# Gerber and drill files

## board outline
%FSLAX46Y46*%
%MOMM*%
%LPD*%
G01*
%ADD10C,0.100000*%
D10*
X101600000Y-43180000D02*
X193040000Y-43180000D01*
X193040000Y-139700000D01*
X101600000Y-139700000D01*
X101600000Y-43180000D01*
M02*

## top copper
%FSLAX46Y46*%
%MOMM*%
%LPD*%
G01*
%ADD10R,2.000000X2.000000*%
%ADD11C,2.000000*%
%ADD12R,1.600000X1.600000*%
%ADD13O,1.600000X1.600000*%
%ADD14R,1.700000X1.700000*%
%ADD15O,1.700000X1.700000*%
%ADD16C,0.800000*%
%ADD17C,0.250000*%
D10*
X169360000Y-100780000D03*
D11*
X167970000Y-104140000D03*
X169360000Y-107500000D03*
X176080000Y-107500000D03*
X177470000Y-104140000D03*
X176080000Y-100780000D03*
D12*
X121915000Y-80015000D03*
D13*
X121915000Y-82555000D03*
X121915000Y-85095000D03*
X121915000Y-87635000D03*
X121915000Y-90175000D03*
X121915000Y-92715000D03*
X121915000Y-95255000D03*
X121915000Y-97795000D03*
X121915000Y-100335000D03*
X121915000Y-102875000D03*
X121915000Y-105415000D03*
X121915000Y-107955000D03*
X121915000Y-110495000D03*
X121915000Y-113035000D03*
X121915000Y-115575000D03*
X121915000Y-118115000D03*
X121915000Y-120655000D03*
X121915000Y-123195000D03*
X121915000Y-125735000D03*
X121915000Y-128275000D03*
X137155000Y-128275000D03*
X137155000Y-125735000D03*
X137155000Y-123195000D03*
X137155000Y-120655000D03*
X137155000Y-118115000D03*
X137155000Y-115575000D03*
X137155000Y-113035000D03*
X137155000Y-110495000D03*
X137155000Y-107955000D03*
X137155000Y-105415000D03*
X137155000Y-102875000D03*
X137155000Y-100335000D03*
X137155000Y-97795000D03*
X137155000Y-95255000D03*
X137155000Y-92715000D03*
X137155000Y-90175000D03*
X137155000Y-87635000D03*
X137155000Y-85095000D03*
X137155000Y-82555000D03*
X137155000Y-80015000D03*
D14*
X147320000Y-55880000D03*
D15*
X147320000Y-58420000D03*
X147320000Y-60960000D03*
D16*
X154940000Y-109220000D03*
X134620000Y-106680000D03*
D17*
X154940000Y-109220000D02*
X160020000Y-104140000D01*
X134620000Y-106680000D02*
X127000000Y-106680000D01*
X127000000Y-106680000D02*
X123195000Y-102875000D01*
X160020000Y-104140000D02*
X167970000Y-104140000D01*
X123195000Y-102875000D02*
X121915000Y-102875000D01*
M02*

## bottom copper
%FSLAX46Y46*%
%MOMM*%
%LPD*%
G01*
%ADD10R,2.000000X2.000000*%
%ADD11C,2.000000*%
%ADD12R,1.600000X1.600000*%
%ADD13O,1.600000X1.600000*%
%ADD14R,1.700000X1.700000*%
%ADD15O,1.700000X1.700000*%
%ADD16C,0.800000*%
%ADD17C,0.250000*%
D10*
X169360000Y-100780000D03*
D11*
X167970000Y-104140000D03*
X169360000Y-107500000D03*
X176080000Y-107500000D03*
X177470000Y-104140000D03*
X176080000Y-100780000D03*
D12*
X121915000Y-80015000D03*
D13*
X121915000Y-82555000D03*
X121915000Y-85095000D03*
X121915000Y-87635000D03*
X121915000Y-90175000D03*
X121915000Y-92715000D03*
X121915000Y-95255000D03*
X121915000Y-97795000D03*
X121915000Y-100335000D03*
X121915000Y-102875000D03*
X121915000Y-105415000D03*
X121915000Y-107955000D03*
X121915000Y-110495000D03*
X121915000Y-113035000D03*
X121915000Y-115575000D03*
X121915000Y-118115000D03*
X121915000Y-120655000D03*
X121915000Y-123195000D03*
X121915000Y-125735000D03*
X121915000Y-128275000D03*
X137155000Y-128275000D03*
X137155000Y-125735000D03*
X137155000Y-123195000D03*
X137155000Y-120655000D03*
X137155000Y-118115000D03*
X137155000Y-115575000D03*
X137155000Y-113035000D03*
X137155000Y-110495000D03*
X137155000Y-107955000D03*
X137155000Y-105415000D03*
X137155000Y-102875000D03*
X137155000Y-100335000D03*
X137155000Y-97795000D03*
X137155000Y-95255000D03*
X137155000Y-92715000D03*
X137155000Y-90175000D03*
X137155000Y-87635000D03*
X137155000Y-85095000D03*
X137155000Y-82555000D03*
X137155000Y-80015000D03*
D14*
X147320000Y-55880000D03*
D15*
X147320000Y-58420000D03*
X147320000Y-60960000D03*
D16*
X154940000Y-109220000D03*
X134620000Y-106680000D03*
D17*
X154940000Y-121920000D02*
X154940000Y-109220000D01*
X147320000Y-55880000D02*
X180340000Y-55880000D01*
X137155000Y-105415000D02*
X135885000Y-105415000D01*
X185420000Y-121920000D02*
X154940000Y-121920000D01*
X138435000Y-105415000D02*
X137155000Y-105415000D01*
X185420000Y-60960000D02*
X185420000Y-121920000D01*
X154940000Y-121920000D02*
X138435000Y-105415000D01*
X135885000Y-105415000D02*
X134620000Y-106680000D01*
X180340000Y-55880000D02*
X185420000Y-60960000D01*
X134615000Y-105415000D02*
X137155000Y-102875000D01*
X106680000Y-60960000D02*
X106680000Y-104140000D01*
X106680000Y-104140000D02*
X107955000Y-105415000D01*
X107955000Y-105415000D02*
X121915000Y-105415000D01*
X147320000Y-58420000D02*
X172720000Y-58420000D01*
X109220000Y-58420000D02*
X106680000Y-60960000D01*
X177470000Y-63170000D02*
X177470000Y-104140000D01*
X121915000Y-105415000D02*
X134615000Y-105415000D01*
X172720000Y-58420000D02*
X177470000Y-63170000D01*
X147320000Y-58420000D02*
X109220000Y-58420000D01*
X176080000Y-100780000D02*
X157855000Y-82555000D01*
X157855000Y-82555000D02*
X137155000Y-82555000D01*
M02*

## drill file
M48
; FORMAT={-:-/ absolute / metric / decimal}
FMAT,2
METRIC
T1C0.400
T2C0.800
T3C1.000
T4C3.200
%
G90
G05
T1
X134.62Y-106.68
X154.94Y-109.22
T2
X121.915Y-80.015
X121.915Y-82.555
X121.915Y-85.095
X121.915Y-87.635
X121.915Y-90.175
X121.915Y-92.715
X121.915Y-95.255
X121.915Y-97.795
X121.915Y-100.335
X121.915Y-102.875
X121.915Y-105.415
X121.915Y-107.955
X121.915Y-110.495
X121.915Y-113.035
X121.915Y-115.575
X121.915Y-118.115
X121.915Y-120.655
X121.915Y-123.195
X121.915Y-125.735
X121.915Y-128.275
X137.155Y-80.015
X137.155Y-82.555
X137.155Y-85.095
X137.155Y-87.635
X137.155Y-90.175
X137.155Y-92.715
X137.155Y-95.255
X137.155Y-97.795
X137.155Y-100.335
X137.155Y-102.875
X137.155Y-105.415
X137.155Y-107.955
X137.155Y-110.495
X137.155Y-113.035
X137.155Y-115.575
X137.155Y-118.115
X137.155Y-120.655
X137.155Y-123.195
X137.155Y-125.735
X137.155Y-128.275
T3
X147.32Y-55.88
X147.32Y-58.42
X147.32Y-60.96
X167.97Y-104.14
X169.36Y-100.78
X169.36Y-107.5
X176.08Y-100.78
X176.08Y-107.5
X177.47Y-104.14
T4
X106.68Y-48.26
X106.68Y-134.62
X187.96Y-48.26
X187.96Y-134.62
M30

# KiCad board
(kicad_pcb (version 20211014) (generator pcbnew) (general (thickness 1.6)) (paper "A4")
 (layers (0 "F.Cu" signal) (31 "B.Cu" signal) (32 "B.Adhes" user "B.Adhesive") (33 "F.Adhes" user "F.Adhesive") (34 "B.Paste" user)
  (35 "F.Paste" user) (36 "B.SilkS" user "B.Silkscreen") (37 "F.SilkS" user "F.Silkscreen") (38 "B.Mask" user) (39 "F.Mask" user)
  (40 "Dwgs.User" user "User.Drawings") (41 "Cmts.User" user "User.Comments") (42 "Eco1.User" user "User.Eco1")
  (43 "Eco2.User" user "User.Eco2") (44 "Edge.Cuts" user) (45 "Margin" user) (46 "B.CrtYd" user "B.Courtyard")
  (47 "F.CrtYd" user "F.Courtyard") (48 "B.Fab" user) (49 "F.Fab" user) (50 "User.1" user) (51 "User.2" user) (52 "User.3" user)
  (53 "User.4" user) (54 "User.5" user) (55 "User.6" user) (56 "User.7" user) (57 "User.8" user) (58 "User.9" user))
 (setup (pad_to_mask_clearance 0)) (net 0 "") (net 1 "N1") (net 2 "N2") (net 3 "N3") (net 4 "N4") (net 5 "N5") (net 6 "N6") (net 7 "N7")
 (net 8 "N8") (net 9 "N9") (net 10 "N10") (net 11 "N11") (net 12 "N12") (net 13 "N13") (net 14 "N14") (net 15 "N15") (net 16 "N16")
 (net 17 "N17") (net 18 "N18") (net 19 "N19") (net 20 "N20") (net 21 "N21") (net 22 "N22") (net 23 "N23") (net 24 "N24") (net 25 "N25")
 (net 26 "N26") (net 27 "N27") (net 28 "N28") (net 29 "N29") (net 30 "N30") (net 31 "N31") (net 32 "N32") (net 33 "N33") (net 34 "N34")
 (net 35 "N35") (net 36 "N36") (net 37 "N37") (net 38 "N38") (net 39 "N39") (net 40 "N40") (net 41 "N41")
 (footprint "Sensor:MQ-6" (layer "F.Cu") (at 169.36 100.78)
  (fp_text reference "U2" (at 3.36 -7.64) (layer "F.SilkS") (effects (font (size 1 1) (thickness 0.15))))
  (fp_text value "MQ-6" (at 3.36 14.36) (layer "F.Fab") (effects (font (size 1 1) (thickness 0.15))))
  (pad "1" thru_hole rect (at 0 0) (size 2 2) (drill 1) (layers *.Cu *.Mask) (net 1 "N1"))
  (pad "2" thru_hole circle (at -1.39 3.36) (size 2 2) (drill 1) (layers *.Cu *.Mask) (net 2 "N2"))
  (pad "3" thru_hole circle (at 0 6.72 90) (size 2 2) (drill 1) (layers *.Cu *.Mask) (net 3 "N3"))
  (pad "4" thru_hole circle (at 6.72 6.72 180) (size 2 2) (drill 1) (layers *.Cu *.Mask) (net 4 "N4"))
  (pad "5" thru_hole circle (at 8.11 3.36) (size 2 2) (drill 1) (layers *.Cu *.Mask) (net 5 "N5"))
  (pad "6" thru_hole circle (at 6.72 0 270) (size 2 2) (drill 1) (layers *.Cu *.Mask) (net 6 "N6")))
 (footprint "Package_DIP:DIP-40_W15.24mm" (layer "F.Cu") (at 121.915 80.015)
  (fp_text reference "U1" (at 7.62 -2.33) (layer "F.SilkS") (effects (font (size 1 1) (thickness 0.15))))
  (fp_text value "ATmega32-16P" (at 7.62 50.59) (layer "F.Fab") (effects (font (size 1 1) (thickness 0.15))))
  (pad "1" thru_hole rect (at 0 0) (size 1.6 1.6) (drill 0.8) (layers *.Cu *.Mask) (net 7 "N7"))
  (pad "2" thru_hole oval (at 0 2.54) (size 1.6 1.6) (drill 0.8) (layers *.Cu *.Mask) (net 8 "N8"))
  (pad "3" thru_hole oval (at 0 5.08) (size 1.6 1.6) (drill 0.8) (layers *.Cu *.Mask) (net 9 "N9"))
  (pad "4" thru_hole oval (at 0 7.62) (size 1.6 1.6) (drill 0.8) (layers *.Cu *.Mask) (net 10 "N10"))
  (pad "5" thru_hole oval (at 0 10.16) (size 1.6 1.6) (drill 0.8) (layers *.Cu *.Mask) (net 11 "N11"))
  (pad "6" thru_hole oval (at 0 12.7) (size 1.6 1.6) (drill 0.8) (layers *.Cu *.Mask) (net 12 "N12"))
  (pad "7" thru_hole oval (at 0 15.24) (size 1.6 1.6) (drill 0.8) (layers *.Cu *.Mask) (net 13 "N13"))
  (pad "8" thru_hole oval (at 0 17.78) (size 1.6 1.6) (drill 0.8) (layers *.Cu *.Mask) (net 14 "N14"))
  (pad "9" thru_hole oval (at 0 20.32) (size 1.6 1.6) (drill 0.8) (layers *.Cu *.Mask) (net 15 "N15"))
  (pad "10" thru_hole oval (at 0 22.86) (size 1.6 1.6) (drill 0.8) (layers *.Cu *.Mask) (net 2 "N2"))
  (pad "11" thru_hole oval (at 0 25.4) (size 1.6 1.6) (drill 0.8) (layers *.Cu *.Mask) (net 5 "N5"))
  (pad "12" thru_hole oval (at 0 27.94) (size 1.6 1.6) (drill 0.8) (layers *.Cu *.Mask) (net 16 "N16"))
  (pad "13" thru_hole oval (at 0 30.48) (size 1.6 1.6) (drill 0.8) (layers *.Cu *.Mask) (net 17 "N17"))
  (pad "14" thru_hole oval (at 0 33.02) (size 1.6 1.6) (drill 0.8) (layers *.Cu *.Mask) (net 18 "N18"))
  (pad "15" thru_hole oval (at 0 35.56) (size 1.6 1.6) (drill 0.8) (layers *.Cu *.Mask) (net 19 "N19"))
  (pad "16" thru_hole oval (at 0 38.1) (size 1.6 1.6) (drill 0.8) (layers *.Cu *.Mask) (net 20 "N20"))
  (pad "17" thru_hole oval (at 0 40.64) (size 1.6 1.6) (drill 0.8) (layers *.Cu *.Mask) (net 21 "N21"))
  (pad "18" thru_hole oval (at 0 43.18) (size 1.6 1.6) (drill 0.8) (layers *.Cu *.Mask) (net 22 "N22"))
  (pad "19" thru_hole oval (at 0 45.72) (size 1.6 1.6) (drill 0.8) (layers *.Cu *.Mask) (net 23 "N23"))
  (pad "20" thru_hole oval (at 0 48.26) (size 1.6 1.6) (drill 0.8) (layers *.Cu *.Mask) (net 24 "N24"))
  (pad "21" thru_hole oval (at 15.24 48.26) (size 1.6 1.6) (drill 0.8) (layers *.Cu *.Mask) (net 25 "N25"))
  (pad "22" thru_hole oval (at 15.24 45.72) (size 1.6 1.6) (drill 0.8) (layers *.Cu *.Mask) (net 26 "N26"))
  (pad "23" thru_hole oval (at 15.24 43.18) (size 1.6 1.6) (drill 0.8) (layers *.Cu *.Mask) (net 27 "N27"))
  (pad "24" thru_hole oval (at 15.24 40.64) (size 1.6 1.6) (drill 0.8) (layers *.Cu *.Mask) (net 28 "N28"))
  (pad "25" thru_hole oval (at 15.24 38.1) (size 1.6 1.6) (drill 0.8) (layers *.Cu *.Mask) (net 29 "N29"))
  (pad "26" thru_hole oval (at 15.24 35.56) (size 1.6 1.6) (drill 0.8) (layers *.Cu *.Mask) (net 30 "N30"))
  (pad "27" thru_hole oval (at 15.24 33.02) (size 1.6 1.6) (drill 0.8) (layers *.Cu *.Mask) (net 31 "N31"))
  (pad "28" thru_hole oval (at 15.24 30.48) (size 1.6 1.6) (drill 0.8) (layers *.Cu *.Mask) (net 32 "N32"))
  (pad "29" thru_hole oval (at 15.24 27.94) (size 1.6 1.6) (drill 0.8) (layers *.Cu *.Mask) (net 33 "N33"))
  (pad "30" thru_hole oval (at 15.24 25.4) (size 1.6 1.6) (drill 0.8) (layers *.Cu *.Mask) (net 2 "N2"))
  (pad "31" thru_hole oval (at 15.24 22.86) (size 1.6 1.6) (drill 0.8) (layers *.Cu *.Mask) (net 5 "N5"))
  (pad "32" thru_hole oval (at 15.24 20.32) (size 1.6 1.6) (drill 0.8) (layers *.Cu *.Mask) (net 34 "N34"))
  (pad "33" thru_hole oval (at 15.24 17.78) (size 1.6 1.6) (drill 0.8) (layers *.Cu *.Mask) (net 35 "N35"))
  (pad "34" thru_hole oval (at 15.24 15.24) (size 1.6 1.6) (drill 0.8) (layers *.Cu *.Mask) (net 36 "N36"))
  (pad "35" thru_hole oval (at 15.24 12.7) (size 1.6 1.6) (drill 0.8) (layers *.Cu *.Mask) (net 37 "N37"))
  (pad "36" thru_hole oval (at 15.24 10.16) (size 1.6 1.6) (drill 0.8) (layers *.Cu *.Mask) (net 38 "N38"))
  (pad "37" thru_hole oval (at 15.24 7.62) (size 1.6 1.6) (drill 0.8) (layers *.Cu *.Mask) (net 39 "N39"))
  (pad "38" thru_hole oval (at 15.24 5.08) (size 1.6 1.6) (drill 0.8) (layers *.Cu *.Mask) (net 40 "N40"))
  (pad "39" thru_hole oval (at 15.24 2.54) (size 1.6 1.6) (drill 0.8) (layers *.Cu *.Mask) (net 6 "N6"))
  (pad "40" thru_hole oval (at 15.24 0) (size 1.6 1.6) (drill 0.8) (layers *.Cu *.Mask) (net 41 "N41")))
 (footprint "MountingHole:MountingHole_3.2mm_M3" (layer "F.Cu") (at 106.68 48.26)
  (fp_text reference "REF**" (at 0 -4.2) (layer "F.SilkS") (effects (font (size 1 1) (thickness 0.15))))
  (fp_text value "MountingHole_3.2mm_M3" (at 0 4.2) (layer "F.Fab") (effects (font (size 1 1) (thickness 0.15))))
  (pad "" np_thru_hole circle (at 0 0) (size 3.2 3.2) (drill 3.2) (layers *.Cu *.Mask)))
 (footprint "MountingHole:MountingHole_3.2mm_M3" (layer "F.Cu") (at 187.96 134.62)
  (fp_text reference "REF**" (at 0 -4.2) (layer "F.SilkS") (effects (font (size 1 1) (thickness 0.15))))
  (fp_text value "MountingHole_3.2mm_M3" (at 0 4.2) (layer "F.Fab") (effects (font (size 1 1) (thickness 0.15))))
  (pad "" np_thru_hole circle (at 0 0) (size 3.2 3.2) (drill 3.2) (layers *.Cu *.Mask)))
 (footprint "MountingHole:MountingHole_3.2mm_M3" (layer "F.Cu") (at 187.96 48.26)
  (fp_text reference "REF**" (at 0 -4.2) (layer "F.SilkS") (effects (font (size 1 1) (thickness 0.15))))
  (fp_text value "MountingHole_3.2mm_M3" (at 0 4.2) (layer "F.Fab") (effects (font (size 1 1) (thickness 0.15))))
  (pad "" np_thru_hole circle (at 0 0) (size 3.2 3.2) (drill 3.2) (layers *.Cu *.Mask)))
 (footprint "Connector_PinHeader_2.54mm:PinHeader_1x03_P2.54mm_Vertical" (layer "F.Cu") (at 147.32 55.88)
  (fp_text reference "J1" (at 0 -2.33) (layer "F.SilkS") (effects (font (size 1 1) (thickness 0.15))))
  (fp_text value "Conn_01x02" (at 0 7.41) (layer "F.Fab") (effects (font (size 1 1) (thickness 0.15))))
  (pad "1" thru_hole rect (at 0 0) (size 1.7 1.7) (drill 1) (layers *.Cu *.Mask) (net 2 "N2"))
  (pad "2" thru_hole oval (at 0 2.54) (size 1.7 1.7) (drill 1) (layers *.Cu *.Mask) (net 5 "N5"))
  (pad "3" thru_hole oval (at 0 5.08) (size 1.7 1.7) (drill 1) (layers *.Cu *.Mask)))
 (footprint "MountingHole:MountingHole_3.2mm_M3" (layer "F.Cu") (at 106.68 134.62)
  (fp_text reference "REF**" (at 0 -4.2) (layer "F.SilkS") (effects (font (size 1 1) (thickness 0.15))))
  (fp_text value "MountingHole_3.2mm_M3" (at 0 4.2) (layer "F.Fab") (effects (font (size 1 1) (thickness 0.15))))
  (pad "" np_thru_hole circle (at 0 0) (size 3.2 3.2) (drill 3.2) (layers *.Cu *.Mask)))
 (gr_rect (start 101.6 43.18) (end 193.04 139.7) (layer "Edge.Cuts") (width 0.1) (fill none))
 (segment (start 154.94 109.22) (end 160.02 104.14) (width 0.25) (layer "F.Cu") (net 2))
 (segment (start 134.62 106.68) (end 127 106.68) (width 0.25) (layer "F.Cu") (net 2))
 (segment (start 127 106.68) (end 123.195 102.875) (width 0.25) (layer "F.Cu") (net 2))
 (segment (start 160.02 104.14) (end 167.97 104.14) (width 0.25) (layer "F.Cu") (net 2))
 (segment (start 123.195 102.875) (end 121.915 102.875) (width 0.25) (layer "F.Cu") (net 2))
 (via (at 154.94 109.22) (size 0.8) (drill 0.4) (layers "F.Cu" "B.Cu") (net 2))
 (via (at 134.62 106.68) (size 0.8) (drill 0.4) (layers "F.Cu" "B.Cu") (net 2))
 (segment (start 154.94 121.92) (end 154.94 109.22) (width 0.25) (layer "B.Cu") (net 2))
 (segment (start 147.32 55.88) (end 180.34 55.88) (width 0.25) (layer "B.Cu") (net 2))
 (segment (start 137.155 105.415) (end 135.885 105.415) (width 0.25) (layer "B.Cu") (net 2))
 (segment (start 185.42 121.92) (end 154.94 121.92) (width 0.25) (layer "B.Cu") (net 2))
 (segment (start 138.435 105.415) (end 137.155 105.415) (width 0.25) (layer "B.Cu") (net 2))
 (segment (start 185.42 60.96) (end 185.42 121.92) (width 0.25) (layer "B.Cu") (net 2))
 (segment (start 154.94 121.92) (end 138.435 105.415) (width 0.25) (layer "B.Cu") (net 2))
 (segment (start 135.885 105.415) (end 134.62 106.68) (width 0.25) (layer "B.Cu") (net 2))
 (segment (start 180.34 55.88) (end 185.42 60.96) (width 0.25) (layer "B.Cu") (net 2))
 (segment (start 134.615 105.415) (end 137.155 102.875) (width 0.25) (layer "B.Cu") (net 5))
 (segment (start 106.68 60.96) (end 106.68 104.14) (width 0.25) (layer "B.Cu") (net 5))
 (segment (start 106.68 104.14) (end 107.955 105.415) (width 0.25) (layer "B.Cu") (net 5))
 (segment (start 107.955 105.415) (end 121.915 105.415) (width 0.25) (layer "B.Cu") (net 5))
 (segment (start 147.32 58.42) (end 172.72 58.42) (width 0.25) (layer "B.Cu") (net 5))
 (segment (start 109.22 58.42) (end 106.68 60.96) (width 0.25) (layer "B.Cu") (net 5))
 (segment (start 177.47 63.17) (end 177.47 104.14) (width 0.25) (layer "B.Cu") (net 5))
 (segment (start 121.915 105.415) (end 134.615 105.415) (width 0.25) (layer "B.Cu") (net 5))
 (segment (start 172.72 58.42) (end 177.47 63.17) (width 0.25) (layer "B.Cu") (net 5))
 (segment (start 147.32 58.42) (end 109.22 58.42) (width 0.25) (layer "B.Cu") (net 5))
 (segment (start 176.08 100.78) (end 157.855 82.555) (width 0.25) (layer "B.Cu") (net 6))
 (segment (start 157.855 82.555) (end 137.155 82.555) (width 0.25) (layer "B.Cu") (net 6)))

